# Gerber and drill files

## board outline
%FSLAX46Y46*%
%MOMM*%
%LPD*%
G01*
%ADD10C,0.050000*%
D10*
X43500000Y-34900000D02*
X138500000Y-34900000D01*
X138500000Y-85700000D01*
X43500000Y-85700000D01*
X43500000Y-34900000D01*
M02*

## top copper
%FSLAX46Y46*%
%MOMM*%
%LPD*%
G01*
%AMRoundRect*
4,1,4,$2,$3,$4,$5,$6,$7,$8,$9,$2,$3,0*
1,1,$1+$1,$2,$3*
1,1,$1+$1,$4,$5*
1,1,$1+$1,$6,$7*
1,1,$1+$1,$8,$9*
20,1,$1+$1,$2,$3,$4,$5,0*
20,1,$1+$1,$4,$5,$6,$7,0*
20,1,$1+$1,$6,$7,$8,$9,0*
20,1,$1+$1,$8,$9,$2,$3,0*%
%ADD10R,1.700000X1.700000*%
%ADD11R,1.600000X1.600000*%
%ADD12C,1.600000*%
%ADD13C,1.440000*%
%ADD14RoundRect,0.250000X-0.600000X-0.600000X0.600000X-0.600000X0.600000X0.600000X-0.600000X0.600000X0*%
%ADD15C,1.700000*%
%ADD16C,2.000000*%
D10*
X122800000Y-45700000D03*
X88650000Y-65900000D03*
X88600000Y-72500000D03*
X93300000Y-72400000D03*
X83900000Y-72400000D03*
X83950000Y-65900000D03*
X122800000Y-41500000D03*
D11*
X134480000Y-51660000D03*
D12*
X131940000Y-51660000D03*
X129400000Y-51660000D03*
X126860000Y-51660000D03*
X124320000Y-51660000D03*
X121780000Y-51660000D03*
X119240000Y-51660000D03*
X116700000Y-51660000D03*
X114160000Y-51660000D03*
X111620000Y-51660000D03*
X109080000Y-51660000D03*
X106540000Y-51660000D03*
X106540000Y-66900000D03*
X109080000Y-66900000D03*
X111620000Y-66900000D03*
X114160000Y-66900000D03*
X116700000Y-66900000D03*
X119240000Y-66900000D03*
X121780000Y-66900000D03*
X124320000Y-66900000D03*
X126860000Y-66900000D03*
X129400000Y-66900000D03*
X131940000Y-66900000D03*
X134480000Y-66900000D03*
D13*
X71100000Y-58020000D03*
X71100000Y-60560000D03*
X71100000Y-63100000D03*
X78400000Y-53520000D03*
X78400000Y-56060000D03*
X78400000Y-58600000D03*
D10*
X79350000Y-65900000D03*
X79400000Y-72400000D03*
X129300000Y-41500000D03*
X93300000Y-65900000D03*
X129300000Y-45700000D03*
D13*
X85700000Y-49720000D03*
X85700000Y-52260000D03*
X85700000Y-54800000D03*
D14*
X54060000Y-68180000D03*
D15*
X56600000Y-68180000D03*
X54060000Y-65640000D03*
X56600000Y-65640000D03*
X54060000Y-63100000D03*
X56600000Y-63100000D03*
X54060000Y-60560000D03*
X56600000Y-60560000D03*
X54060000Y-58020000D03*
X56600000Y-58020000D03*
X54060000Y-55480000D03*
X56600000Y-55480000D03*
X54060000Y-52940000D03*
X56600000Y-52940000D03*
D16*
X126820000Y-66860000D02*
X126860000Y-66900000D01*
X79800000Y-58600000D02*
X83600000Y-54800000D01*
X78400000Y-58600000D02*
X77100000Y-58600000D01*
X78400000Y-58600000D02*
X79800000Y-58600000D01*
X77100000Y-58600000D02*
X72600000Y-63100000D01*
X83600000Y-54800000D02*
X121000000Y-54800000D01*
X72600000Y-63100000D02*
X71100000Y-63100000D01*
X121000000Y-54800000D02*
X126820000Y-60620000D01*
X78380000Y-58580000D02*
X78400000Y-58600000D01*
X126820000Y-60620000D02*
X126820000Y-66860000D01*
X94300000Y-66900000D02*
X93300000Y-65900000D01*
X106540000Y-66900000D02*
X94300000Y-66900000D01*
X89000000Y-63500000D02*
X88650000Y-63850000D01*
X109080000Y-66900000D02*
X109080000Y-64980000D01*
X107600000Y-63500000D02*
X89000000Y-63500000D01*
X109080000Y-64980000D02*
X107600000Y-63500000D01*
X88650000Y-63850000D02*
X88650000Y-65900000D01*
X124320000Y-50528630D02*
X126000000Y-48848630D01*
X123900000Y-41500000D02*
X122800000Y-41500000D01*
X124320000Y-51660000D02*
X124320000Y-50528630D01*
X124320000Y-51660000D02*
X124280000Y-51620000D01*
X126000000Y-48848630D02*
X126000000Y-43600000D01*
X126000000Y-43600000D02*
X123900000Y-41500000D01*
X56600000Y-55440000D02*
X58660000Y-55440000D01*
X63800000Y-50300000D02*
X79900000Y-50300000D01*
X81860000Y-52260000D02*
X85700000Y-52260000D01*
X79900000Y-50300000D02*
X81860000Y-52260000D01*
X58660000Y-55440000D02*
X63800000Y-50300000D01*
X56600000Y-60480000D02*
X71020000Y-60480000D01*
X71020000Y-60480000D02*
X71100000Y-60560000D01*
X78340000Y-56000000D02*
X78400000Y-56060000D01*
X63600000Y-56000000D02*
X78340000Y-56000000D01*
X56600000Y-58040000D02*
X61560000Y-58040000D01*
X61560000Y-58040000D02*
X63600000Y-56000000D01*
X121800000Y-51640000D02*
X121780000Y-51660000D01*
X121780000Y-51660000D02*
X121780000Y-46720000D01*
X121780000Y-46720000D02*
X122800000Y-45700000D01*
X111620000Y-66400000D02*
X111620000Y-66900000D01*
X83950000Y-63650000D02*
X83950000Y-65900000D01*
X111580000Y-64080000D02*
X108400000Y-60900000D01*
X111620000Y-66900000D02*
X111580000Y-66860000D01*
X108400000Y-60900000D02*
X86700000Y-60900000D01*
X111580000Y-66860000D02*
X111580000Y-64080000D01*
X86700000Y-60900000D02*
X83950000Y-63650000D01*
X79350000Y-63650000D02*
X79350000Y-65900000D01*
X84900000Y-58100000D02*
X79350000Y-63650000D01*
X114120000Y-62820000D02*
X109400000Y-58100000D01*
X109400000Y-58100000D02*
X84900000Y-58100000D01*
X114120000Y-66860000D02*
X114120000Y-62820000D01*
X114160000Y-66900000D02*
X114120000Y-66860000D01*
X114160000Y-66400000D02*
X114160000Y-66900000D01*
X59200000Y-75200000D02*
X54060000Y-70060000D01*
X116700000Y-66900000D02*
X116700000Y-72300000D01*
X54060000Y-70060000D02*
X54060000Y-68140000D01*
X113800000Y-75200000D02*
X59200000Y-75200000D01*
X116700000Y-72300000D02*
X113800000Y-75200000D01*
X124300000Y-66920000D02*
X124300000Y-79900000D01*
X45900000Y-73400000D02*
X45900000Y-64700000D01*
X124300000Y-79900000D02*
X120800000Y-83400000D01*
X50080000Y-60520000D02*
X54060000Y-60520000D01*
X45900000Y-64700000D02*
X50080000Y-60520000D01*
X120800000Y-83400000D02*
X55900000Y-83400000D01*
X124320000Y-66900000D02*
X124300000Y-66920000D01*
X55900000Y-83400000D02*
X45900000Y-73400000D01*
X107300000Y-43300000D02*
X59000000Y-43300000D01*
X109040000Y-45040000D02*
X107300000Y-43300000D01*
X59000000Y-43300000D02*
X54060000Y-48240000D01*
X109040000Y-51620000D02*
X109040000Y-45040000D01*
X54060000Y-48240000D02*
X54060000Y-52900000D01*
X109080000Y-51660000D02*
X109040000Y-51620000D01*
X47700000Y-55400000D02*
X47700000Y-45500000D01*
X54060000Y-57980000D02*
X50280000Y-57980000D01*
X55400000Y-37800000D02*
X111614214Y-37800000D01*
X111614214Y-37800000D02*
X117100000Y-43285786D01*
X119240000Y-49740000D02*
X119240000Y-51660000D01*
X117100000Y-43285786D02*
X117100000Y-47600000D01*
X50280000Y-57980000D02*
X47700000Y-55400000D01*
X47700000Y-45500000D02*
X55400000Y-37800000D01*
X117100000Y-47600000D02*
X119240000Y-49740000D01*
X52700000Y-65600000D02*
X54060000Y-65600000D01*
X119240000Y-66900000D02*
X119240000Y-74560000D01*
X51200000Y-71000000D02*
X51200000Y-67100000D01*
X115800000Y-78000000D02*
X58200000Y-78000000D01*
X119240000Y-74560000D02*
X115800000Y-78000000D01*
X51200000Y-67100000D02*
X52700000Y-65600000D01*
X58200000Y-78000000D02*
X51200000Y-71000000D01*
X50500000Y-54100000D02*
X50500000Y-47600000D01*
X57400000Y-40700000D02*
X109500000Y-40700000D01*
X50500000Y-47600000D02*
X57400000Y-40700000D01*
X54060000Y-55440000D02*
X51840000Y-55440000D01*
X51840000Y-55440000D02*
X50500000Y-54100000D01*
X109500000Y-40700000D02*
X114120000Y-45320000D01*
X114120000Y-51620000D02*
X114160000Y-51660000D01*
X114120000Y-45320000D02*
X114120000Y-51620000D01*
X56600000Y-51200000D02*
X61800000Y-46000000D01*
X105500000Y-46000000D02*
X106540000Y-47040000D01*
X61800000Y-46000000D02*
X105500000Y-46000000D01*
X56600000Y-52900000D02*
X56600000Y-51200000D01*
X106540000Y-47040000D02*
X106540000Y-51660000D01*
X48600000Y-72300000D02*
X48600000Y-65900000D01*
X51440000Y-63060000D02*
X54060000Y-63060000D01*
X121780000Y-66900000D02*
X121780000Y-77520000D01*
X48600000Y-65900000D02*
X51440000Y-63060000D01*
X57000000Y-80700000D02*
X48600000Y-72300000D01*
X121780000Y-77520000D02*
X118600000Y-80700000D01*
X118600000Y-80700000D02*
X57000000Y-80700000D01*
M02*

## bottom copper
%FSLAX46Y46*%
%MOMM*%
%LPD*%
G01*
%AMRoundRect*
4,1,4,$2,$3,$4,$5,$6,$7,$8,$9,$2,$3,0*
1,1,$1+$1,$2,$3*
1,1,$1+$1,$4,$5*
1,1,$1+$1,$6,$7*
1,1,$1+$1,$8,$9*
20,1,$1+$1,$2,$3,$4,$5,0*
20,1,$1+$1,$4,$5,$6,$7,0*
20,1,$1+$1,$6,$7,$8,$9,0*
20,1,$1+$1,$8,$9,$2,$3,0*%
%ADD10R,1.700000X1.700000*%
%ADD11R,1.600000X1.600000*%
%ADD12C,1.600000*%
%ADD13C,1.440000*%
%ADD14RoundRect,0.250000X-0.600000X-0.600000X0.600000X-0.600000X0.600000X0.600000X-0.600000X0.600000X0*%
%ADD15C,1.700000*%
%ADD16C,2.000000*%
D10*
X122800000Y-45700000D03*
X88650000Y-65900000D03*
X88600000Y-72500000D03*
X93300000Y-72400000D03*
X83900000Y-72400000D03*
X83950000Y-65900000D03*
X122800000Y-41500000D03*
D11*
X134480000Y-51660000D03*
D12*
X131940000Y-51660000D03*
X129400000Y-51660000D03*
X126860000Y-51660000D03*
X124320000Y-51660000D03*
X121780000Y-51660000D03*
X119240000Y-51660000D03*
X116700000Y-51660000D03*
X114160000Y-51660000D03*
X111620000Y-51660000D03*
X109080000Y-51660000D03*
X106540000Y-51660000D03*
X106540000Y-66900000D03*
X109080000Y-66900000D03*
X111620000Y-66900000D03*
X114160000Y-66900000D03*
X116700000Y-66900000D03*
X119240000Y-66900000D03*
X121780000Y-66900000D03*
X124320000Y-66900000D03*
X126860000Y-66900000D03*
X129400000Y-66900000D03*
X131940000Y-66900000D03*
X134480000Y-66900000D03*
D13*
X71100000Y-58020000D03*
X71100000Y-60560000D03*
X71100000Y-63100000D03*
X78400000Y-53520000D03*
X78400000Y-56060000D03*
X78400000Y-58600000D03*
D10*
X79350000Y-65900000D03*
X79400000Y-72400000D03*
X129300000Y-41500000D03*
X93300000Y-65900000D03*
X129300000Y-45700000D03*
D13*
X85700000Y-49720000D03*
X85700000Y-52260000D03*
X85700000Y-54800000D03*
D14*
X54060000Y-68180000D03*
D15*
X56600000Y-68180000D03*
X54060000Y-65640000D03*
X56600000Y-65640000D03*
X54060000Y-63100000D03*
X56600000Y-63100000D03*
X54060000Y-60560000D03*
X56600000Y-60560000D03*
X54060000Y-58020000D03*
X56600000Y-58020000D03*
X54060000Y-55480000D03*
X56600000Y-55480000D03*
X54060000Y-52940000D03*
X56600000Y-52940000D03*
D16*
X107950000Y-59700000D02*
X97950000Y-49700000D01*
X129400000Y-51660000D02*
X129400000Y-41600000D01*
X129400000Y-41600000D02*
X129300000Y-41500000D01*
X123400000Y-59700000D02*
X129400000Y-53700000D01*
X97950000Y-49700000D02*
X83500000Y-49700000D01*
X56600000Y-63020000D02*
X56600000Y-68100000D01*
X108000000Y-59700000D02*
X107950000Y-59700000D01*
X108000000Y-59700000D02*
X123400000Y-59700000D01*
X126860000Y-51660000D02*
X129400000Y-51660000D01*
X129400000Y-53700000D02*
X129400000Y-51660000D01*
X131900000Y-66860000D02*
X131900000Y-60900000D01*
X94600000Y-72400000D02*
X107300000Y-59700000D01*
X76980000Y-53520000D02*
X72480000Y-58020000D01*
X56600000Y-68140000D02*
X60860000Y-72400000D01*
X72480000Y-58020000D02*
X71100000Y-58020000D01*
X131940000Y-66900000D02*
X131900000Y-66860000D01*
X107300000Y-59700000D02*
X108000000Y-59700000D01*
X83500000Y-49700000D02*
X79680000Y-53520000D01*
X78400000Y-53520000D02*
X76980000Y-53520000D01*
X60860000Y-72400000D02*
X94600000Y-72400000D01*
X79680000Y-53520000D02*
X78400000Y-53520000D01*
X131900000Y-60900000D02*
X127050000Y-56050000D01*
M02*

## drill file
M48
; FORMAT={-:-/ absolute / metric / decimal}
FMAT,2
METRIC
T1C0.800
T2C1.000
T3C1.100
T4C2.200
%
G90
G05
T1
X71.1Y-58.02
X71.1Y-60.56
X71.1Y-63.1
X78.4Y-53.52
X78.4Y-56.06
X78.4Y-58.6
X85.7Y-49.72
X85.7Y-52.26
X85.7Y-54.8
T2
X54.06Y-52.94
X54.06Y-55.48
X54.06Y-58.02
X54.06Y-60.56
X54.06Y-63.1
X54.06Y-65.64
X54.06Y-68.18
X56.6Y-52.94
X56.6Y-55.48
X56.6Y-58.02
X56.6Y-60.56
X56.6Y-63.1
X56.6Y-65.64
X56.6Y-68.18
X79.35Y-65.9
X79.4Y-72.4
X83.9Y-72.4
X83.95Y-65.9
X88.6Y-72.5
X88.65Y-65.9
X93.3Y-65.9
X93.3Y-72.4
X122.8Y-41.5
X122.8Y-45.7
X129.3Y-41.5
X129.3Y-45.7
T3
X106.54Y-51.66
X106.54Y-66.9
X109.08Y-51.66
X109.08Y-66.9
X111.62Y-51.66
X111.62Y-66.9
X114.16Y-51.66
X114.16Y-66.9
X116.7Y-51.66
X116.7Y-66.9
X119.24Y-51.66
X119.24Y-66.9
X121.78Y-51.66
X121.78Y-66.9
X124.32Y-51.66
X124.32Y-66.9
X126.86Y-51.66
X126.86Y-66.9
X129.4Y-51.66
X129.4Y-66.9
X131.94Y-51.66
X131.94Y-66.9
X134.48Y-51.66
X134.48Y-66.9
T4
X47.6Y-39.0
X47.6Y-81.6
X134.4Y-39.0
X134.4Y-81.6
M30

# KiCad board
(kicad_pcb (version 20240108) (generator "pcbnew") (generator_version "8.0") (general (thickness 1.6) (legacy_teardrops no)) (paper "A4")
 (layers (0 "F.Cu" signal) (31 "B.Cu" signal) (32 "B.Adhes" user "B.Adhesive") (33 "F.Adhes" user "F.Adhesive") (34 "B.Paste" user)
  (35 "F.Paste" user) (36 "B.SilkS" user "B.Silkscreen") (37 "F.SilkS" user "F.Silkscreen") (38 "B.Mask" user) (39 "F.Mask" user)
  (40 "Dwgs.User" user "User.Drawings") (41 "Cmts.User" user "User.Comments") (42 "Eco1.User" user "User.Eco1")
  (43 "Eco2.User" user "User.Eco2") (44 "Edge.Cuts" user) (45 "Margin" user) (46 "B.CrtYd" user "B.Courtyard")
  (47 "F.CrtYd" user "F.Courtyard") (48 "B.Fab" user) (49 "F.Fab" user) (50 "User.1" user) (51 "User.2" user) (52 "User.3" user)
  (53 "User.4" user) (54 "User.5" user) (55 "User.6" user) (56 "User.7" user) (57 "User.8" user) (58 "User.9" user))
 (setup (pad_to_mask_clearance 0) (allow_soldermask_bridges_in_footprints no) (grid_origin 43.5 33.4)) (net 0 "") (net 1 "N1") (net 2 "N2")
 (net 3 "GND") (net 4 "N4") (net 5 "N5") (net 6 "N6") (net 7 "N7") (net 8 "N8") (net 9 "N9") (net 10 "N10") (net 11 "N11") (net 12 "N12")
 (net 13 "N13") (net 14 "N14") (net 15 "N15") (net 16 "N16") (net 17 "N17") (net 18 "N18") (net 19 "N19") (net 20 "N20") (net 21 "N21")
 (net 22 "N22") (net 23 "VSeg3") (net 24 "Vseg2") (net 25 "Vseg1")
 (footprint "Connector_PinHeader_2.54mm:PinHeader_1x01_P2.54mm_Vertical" (layer "F.Cu") (at 122.8 45.7 180)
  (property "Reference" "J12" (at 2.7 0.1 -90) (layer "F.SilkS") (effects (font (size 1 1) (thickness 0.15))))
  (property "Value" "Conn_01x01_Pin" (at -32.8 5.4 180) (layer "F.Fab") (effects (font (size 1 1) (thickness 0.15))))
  (pad "1" thru_hole rect (at 0 0 180) (size 1.7 1.7) (drill 1) (layers "*.Cu" "*.Mask") (remove_unused_layers no) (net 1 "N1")))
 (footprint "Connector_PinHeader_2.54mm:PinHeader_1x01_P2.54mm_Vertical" (layer "F.Cu") (at 88.65 65.9 180)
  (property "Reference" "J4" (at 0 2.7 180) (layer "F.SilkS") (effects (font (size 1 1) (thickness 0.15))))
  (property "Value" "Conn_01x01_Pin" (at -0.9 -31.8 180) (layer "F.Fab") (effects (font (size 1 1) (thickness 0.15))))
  (pad "1" thru_hole rect (at 0 0 180) (size 1.7 1.7) (drill 1) (layers "*.Cu" "*.Mask") (remove_unused_layers no) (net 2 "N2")))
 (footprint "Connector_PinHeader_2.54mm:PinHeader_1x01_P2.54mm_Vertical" (layer "F.Cu") (at 88.6 72.5 180)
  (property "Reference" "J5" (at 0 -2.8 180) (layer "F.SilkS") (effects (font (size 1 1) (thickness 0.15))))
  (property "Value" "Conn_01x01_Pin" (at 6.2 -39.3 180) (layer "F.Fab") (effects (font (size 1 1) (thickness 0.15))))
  (pad "1" thru_hole rect (at 0 0 180) (size 1.7 1.7) (drill 1) (layers "*.Cu" "*.Mask") (remove_unused_layers no) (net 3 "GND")))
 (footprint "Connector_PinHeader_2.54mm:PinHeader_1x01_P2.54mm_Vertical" (layer "F.Cu") (at 93.3 72.4 180)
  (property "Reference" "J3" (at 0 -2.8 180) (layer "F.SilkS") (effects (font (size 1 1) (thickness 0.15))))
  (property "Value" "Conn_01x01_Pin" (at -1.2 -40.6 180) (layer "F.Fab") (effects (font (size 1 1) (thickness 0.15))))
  (pad "1" thru_hole rect (at 0 0 180) (size 1.7 1.7) (drill 1) (layers "*.Cu" "*.Mask") (remove_unused_layers no) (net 3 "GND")))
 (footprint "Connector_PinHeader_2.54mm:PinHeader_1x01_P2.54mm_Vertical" (layer "F.Cu") (at 83.9 72.4 180)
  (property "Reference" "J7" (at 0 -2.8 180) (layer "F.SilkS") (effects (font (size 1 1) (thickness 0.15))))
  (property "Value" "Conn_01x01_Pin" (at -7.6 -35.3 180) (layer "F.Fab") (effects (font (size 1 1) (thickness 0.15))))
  (pad "1" thru_hole rect (at 0 0 180) (size 1.7 1.7) (drill 1) (layers "*.Cu" "*.Mask") (remove_unused_layers no) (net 3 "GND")))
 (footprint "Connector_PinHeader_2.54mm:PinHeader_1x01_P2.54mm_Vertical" (layer "F.Cu") (at 83.95 65.9 180)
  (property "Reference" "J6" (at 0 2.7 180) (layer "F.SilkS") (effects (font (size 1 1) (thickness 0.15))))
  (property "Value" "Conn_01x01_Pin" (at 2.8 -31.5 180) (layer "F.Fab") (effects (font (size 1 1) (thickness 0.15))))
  (pad "1" thru_hole rect (at 0 0 180) (size 1.7 1.7) (drill 1) (layers "*.Cu" "*.Mask") (remove_unused_layers no) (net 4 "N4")))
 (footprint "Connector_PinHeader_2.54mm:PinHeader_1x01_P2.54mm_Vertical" (layer "F.Cu") (at 122.8 41.5 180)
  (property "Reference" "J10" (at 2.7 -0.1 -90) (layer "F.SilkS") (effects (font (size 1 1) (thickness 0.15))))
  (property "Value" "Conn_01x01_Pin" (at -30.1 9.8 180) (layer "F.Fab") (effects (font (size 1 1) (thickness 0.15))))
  (pad "1" thru_hole rect (at 0 0 180) (size 1.7 1.7) (drill 1) (layers "*.Cu" "*.Mask") (remove_unused_layers no) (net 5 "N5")))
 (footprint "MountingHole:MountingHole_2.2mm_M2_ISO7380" (layer "F.Cu") (at 47.6 81.6)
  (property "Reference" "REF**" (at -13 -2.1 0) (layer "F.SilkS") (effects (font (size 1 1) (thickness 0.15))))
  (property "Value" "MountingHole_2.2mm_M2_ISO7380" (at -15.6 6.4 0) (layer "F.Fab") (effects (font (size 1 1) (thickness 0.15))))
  (pad "" np_thru_hole circle (at 0 0) (size 2.2 2.2) (drill 2.2) (layers "*.Cu" "*.Mask")))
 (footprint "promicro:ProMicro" (layer "F.Cu") (at 120.51 59.28 180)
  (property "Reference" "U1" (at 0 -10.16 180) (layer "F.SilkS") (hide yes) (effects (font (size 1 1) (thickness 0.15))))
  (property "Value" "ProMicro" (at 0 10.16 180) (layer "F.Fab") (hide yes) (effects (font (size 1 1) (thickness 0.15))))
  (pad "1" thru_hole rect (at -13.97 7.62 180) (size 1.6 1.6) (drill 1.1) (layers "*.Cu" "*.Mask" "F.SilkS") (remove_unused_layers no)
   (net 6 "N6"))
  (pad "2" thru_hole circle (at -11.43 7.62 180) (size 1.6 1.6) (drill 1.1) (layers "*.Cu" "*.Mask" "F.SilkS") (remove_unused_layers no)
   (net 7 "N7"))
  (pad "3" thru_hole circle (at -8.89 7.62 180) (size 1.6 1.6) (drill 1.1) (layers "*.Cu" "*.Mask" "F.SilkS") (remove_unused_layers no)
   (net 3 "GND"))
  (pad "4" thru_hole circle (at -6.35 7.62 180) (size 1.6 1.6) (drill 1.1) (layers "*.Cu" "*.Mask" "F.SilkS") (remove_unused_layers no)
   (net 3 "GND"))
  (pad "5" thru_hole circle (at -3.81 7.62 180) (size 1.6 1.6) (drill 1.1) (layers "*.Cu" "*.Mask" "F.SilkS") (remove_unused_layers no)
   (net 5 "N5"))
  (pad "6" thru_hole circle (at -1.27 7.62 180) (size 1.6 1.6) (drill 1.1) (layers "*.Cu" "*.Mask" "F.SilkS") (remove_unused_layers no)
   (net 1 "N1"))
  (pad "7" thru_hole circle (at 1.27 7.62 180) (size 1.6 1.6) (drill 1.1) (layers "*.Cu" "*.Mask" "F.SilkS") (remove_unused_layers no)
   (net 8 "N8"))
  (pad "8" thru_hole circle (at 3.81 7.62 180) (size 1.6 1.6) (drill 1.1) (layers "*.Cu" "*.Mask" "F.SilkS") (remove_unused_layers no)
   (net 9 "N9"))
  (pad "9" thru_hole circle (at 6.35 7.62 180) (size 1.6 1.6) (drill 1.1) (layers "*.Cu" "*.Mask" "F.SilkS") (remove_unused_layers no)
   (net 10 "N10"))
  (pad "10" thru_hole circle (at 8.89 7.62 180) (size 1.6 1.6) (drill 1.1) (layers "*.Cu" "*.Mask" "F.SilkS") (remove_unused_layers no)
   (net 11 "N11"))
  (pad "11" thru_hole circle (at 11.43 7.62 180) (size 1.6 1.6) (drill 1.1) (layers "*.Cu" "*.Mask" "F.SilkS") (remove_unused_layers no)
   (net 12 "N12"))
  (pad "12" thru_hole circle (at 13.97 7.62 180) (size 1.6 1.6) (drill 1.1) (layers "*.Cu" "*.Mask" "F.SilkS") (remove_unused_layers no)
   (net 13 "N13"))
  (pad "13" thru_hole circle (at 13.97 -7.62 180) (size 1.6 1.6) (drill 1.1) (layers "*.Cu" "*.Mask" "F.SilkS") (remove_unused_layers no)
   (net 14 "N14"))
  (pad "14" thru_hole circle (at 11.43 -7.62 180) (size 1.6 1.6) (drill 1.1) (layers "*.Cu" "*.Mask" "F.SilkS") (remove_unused_layers no)
   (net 2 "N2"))
  (pad "15" thru_hole circle (at 8.89 -7.62 180) (size 1.6 1.6) (drill 1.1) (layers "*.Cu" "*.Mask" "F.SilkS") (remove_unused_layers no)
   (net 4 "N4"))
  (pad "16" thru_hole circle (at 6.35 -7.62 180) (size 1.6 1.6) (drill 1.1) (layers "*.Cu" "*.Mask" "F.SilkS") (remove_unused_layers no)
   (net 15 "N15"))
  (pad "17" thru_hole circle (at 3.81 -7.62 180) (size 1.6 1.6) (drill 1.1) (layers "*.Cu" "*.Mask" "F.SilkS") (remove_unused_layers no)
   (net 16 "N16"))
  (pad "18" thru_hole circle (at 1.27 -7.62 180) (size 1.6 1.6) (drill 1.1) (layers "*.Cu" "*.Mask" "F.SilkS") (remove_unused_layers no)
   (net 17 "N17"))
  (pad "19" thru_hole circle (at -1.27 -7.62 180) (size 1.6 1.6) (drill 1.1) (layers "*.Cu" "*.Mask" "F.SilkS") (remove_unused_layers no)
   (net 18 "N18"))
  (pad "20" thru_hole circle (at -3.81 -7.62 180) (size 1.6 1.6) (drill 1.1) (layers "*.Cu" "*.Mask" "F.SilkS") (remove_unused_layers no)
   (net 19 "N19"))
  (pad "21" thru_hole circle (at -6.35 -7.62 180) (size 1.6 1.6) (drill 1.1) (layers "*.Cu" "*.Mask" "F.SilkS") (remove_unused_layers no)
   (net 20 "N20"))
  (pad "22" thru_hole circle (at -8.89 -7.62 180) (size 1.6 1.6) (drill 1.1) (layers "*.Cu" "*.Mask" "F.SilkS") (remove_unused_layers no)
   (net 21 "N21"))
  (pad "23" thru_hole circle (at -11.43 -7.62 180) (size 1.6 1.6) (drill 1.1) (layers "*.Cu" "*.Mask" "F.SilkS") (remove_unused_layers no)
   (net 3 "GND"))
  (pad "24" thru_hole circle (at -13.97 -7.62 180) (size 1.6 1.6) (drill 1.1) (layers "*.Cu" "*.Mask" "F.SilkS") (remove_unused_layers no)
   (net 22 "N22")))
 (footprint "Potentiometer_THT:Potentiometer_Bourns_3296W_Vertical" (layer "F.Cu") (at 71.1 58.02 90)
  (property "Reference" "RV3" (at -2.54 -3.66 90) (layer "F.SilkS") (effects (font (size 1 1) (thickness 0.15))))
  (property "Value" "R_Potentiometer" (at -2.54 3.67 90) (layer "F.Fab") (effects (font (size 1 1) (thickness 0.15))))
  (pad "1" thru_hole circle (at 0 0 90) (size 1.44 1.44) (drill 0.8) (layers "*.Cu" "*.Mask") (remove_unused_layers no) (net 3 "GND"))
  (pad "2" thru_hole circle (at -2.54 0 90) (size 1.44 1.44) (drill 0.8) (layers "*.Cu" "*.Mask") (remove_unused_layers no) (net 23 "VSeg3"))
  (pad "3" thru_hole circle (at -5.08 0 90) (size 1.44 1.44) (drill 0.8) (layers "*.Cu" "*.Mask") (remove_unused_layers no) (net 20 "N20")))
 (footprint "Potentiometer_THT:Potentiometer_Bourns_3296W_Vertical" (layer "F.Cu") (at 78.4 53.52 90)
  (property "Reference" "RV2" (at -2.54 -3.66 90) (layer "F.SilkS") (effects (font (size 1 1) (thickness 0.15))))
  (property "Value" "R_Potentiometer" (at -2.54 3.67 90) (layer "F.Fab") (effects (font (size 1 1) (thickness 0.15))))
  (pad "1" thru_hole circle (at 0 0 90) (size 1.44 1.44) (drill 0.8) (layers "*.Cu" "*.Mask") (remove_unused_layers no) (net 3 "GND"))
  (pad "2" thru_hole circle (at -2.54 0 90) (size 1.44 1.44) (drill 0.8) (layers "*.Cu" "*.Mask") (remove_unused_layers no) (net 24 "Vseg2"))
  (pad "3" thru_hole circle (at -5.08 0 90) (size 1.44 1.44) (drill 0.8) (layers "*.Cu" "*.Mask") (remove_unused_layers no) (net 20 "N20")))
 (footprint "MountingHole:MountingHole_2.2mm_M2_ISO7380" (layer "F.Cu") (at 47.6 39)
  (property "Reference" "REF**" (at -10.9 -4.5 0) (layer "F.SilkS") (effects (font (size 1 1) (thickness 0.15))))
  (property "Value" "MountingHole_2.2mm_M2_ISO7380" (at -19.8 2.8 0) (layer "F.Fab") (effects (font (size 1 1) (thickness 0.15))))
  (pad "" np_thru_hole circle (at 0 0) (size 2.2 2.2) (drill 2.2) (layers "*.Cu" "*.Mask")))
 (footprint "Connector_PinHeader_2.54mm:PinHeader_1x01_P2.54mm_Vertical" (layer "F.Cu") (at 79.35 65.9 180)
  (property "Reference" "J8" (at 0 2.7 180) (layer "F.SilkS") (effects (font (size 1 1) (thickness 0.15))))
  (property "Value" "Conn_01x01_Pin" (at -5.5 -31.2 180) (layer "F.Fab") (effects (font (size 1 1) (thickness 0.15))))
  (pad "1" thru_hole rect (at 0 0 180) (size 1.7 1.7) (drill 1) (layers "*.Cu" "*.Mask") (remove_unused_layers no) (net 15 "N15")))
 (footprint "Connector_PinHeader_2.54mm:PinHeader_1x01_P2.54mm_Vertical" (layer "F.Cu") (at 79.4 72.4 180)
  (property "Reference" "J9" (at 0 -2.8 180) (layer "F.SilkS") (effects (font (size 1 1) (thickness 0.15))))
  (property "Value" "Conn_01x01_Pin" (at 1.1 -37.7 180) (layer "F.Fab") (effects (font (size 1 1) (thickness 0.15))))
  (pad "1" thru_hole rect (at 0 0 180) (size 1.7 1.7) (drill 1) (layers "*.Cu" "*.Mask") (remove_unused_layers no) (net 3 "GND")))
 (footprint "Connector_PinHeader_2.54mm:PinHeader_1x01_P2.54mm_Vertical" (layer "F.Cu") (at 129.3 41.5 180)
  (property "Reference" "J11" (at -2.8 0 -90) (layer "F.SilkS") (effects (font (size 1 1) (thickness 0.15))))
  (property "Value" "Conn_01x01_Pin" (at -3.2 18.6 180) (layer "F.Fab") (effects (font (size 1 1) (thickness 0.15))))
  (pad "1" thru_hole rect (at 0 0 180) (size 1.7 1.7) (drill 1) (layers "*.Cu" "*.Mask") (remove_unused_layers no) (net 3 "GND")))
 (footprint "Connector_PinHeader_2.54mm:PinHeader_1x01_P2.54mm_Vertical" (layer "F.Cu") (at 93.3 65.9 180)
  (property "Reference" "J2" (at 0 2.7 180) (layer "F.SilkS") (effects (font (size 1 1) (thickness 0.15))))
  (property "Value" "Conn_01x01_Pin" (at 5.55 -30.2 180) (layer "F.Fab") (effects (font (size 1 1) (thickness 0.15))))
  (pad "1" thru_hole rect (at 0 0 180) (size 1.7 1.7) (drill 1) (layers "*.Cu" "*.Mask") (remove_unused_layers no) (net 14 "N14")))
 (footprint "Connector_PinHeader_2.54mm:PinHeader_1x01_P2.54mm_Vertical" (layer "F.Cu") (at 129.3 45.7 180)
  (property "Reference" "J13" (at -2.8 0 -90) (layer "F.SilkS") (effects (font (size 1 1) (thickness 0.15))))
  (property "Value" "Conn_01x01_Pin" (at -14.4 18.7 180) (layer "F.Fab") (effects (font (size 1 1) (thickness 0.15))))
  (pad "1" thru_hole rect (at 0 0 180) (size 1.7 1.7) (drill 1) (layers "*.Cu" "*.Mask") (remove_unused_layers no) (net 3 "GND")))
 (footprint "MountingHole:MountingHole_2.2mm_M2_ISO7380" (layer "F.Cu") (at 134.4 81.6)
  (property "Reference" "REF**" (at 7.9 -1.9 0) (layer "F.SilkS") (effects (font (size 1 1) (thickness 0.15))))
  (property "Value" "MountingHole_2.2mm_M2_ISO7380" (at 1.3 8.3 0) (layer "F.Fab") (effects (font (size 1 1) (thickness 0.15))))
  (pad "" np_thru_hole circle (at 0 0) (size 2.2 2.2) (drill 2.2) (layers "*.Cu" "*.Mask")))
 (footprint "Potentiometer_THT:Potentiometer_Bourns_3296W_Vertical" (layer "F.Cu") (at 85.7 49.72 90)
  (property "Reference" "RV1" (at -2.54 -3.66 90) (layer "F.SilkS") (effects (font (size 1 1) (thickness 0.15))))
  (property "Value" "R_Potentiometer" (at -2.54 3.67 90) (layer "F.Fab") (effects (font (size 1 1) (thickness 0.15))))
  (pad "1" thru_hole circle (at 0 0 90) (size 1.44 1.44) (drill 0.8) (layers "*.Cu" "*.Mask") (remove_unused_layers no) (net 3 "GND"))
  (pad "2" thru_hole circle (at -2.54 0 90) (size 1.44 1.44) (drill 0.8) (layers "*.Cu" "*.Mask") (remove_unused_layers no) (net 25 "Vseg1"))
  (pad "3" thru_hole circle (at -5.08 0 90) (size 1.44 1.44) (drill 0.8) (layers "*.Cu" "*.Mask") (remove_unused_layers no) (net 20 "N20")))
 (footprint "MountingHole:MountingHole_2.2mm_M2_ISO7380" (layer "F.Cu") (at 134.4 39)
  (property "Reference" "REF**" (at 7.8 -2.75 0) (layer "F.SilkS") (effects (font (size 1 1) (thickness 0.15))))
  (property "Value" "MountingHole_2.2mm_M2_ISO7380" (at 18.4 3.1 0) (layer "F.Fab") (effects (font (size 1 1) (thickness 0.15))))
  (pad "" np_thru_hole circle (at 0 0) (size 2.2 2.2) (drill 2.2) (layers "*.Cu" "*.Mask")))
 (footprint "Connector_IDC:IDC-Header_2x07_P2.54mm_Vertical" (layer "B.Cu") (at 54.06 68.18)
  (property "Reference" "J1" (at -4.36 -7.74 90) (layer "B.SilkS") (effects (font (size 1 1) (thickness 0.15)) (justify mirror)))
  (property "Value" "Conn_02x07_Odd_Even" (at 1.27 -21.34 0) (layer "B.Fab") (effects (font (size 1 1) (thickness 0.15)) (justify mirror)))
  (pad "1" thru_hole roundrect (at 0 0) (size 1.7 1.7) (drill 1) (layers "*.Cu" "*.Mask") (remove_unused_layers no)
   (roundrect_rratio 0.147059) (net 16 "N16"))
  (pad "2" thru_hole circle (at 2.54 0) (size 1.7 1.7) (drill 1) (layers "*.Cu" "*.Mask") (remove_unused_layers no) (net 3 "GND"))
  (pad "3" thru_hole circle (at 0 -2.54) (size 1.7 1.7) (drill 1) (layers "*.Cu" "*.Mask") (remove_unused_layers no) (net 17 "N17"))
  (pad "4" thru_hole circle (at 2.54 -2.54) (size 1.7 1.7) (drill 1) (layers "*.Cu" "*.Mask") (remove_unused_layers no) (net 3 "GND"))
  (pad "5" thru_hole circle (at 0 -5.08) (size 1.7 1.7) (drill 1) (layers "*.Cu" "*.Mask") (remove_unused_layers no) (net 18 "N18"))
  (pad "6" thru_hole circle (at 2.54 -5.08) (size 1.7 1.7) (drill 1) (layers "*.Cu" "*.Mask") (remove_unused_layers no) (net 3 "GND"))
  (pad "7" thru_hole circle (at 0 -7.62) (size 1.7 1.7) (drill 1) (layers "*.Cu" "*.Mask") (remove_unused_layers no) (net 19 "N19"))
  (pad "8" thru_hole circle (at 2.54 -7.62) (size 1.7 1.7) (drill 1) (layers "*.Cu" "*.Mask") (remove_unused_layers no) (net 23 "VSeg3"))
  (pad "9" thru_hole circle (at 0 -10.16) (size 1.7 1.7) (drill 1) (layers "*.Cu" "*.Mask") (remove_unused_layers no) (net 8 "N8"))
  (pad "10" thru_hole circle (at 2.54 -10.16) (size 1.7 1.7) (drill 1) (layers "*.Cu" "*.Mask") (remove_unused_layers no) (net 24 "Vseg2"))
  (pad "11" thru_hole circle (at 0 -12.7) (size 1.7 1.7) (drill 1) (layers "*.Cu" "*.Mask") (remove_unused_layers no) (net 10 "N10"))
  (pad "12" thru_hole circle (at 2.54 -12.7) (size 1.7 1.7) (drill 1) (layers "*.Cu" "*.Mask") (remove_unused_layers no) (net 25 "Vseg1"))
  (pad "13" thru_hole circle (at 0 -15.24) (size 1.7 1.7) (drill 1) (layers "*.Cu" "*.Mask") (remove_unused_layers no) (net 12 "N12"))
  (pad "14" thru_hole circle (at 2.54 -15.24) (size 1.7 1.7) (drill 1) (layers "*.Cu" "*.Mask") (remove_unused_layers no) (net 13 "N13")))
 (gr_rect (start 43.5 34.9) (end 138.5 85.7) (stroke (width 0.05) (type default)) (fill none) (layer "Edge.Cuts"))
 (segment (start 126.82 66.86) (end 126.86 66.9) (width 2) (layer "F.Cu") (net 20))
 (segment (start 79.8 58.6) (end 83.6 54.8) (width 2) (layer "F.Cu") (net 20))
 (segment (start 78.4 58.6) (end 77.1 58.6) (width 2) (layer "F.Cu") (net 20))
 (segment (start 78.4 58.6) (end 79.8 58.6) (width 2) (layer "F.Cu") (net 20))
 (segment (start 77.1 58.6) (end 72.6 63.1) (width 2) (layer "F.Cu") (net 20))
 (segment (start 83.6 54.8) (end 121 54.8) (width 2) (layer "F.Cu") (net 20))
 (segment (start 72.6 63.1) (end 71.1 63.1) (width 2) (layer "F.Cu") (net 20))
 (segment (start 121 54.8) (end 126.82 60.62) (width 2) (layer "F.Cu") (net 20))
 (segment (start 78.38 58.58) (end 78.4 58.6) (width 2) (layer "F.Cu") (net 20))
 (segment (start 126.82 60.62) (end 126.82 66.86) (width 2) (layer "F.Cu") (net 20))
 (segment (start 94.3 66.9) (end 93.3 65.9) (width 2) (layer "F.Cu") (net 14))
 (segment (start 106.54 66.9) (end 94.3 66.9) (width 2) (layer "F.Cu") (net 14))
 (segment (start 89 63.5) (end 88.65 63.85) (width 2) (layer "F.Cu") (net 2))
 (segment (start 109.08 66.9) (end 109.08 64.98) (width 2) (layer "F.Cu") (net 2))
 (segment (start 107.6 63.5) (end 89 63.5) (width 2) (layer "F.Cu") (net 2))
 (segment (start 109.08 64.98) (end 107.6 63.5) (width 2) (layer "F.Cu") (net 2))
 (segment (start 88.65 63.85) (end 88.65 65.9) (width 2) (layer "F.Cu") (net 2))
 (segment (start 124.32 50.52863) (end 126 48.84863) (width 2) (layer "F.Cu") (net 5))
 (segment (start 123.9 41.5) (end 122.8 41.5) (width 2) (layer "F.Cu") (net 5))
 (segment (start 124.32 51.66) (end 124.32 50.52863) (width 2) (layer "F.Cu") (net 5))
 (segment (start 124.32 51.66) (end 124.28 51.62) (width 2) (layer "F.Cu") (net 5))
 (segment (start 126 48.84863) (end 126 43.6) (width 2) (layer "F.Cu") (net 5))
 (segment (start 126 43.6) (end 123.9 41.5) (width 2) (layer "F.Cu") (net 5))
 (segment (start 56.6 55.44) (end 58.66 55.44) (width 2) (layer "F.Cu") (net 25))
 (segment (start 63.8 50.3) (end 79.9 50.3) (width 2) (layer "F.Cu") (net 25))
 (segment (start 81.86 52.26) (end 85.7 52.26) (width 2) (layer "F.Cu") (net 25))
 (segment (start 79.9 50.3) (end 81.86 52.26) (width 2) (layer "F.Cu") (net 25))
 (segment (start 58.66 55.44) (end 63.8 50.3) (width 2) (layer "F.Cu") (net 25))
 (segment (start 56.6 60.48) (end 71.02 60.48) (width 2) (layer "F.Cu") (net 23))
 (segment (start 71.02 60.48) (end 71.1 60.56) (width 2) (layer "F.Cu") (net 23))
 (segment (start 107.95 59.7) (end 97.95 49.7) (width 2) (layer "B.Cu") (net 3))
 (segment (start 129.4 51.66) (end 129.4 41.6) (width 2) (layer "B.Cu") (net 3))
 (segment (start 129.4 41.6) (end 129.3 41.5) (width 2) (layer "B.Cu") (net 3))
 (segment (start 123.4 59.7) (end 129.4 53.7) (width 2) (layer "B.Cu") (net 3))
 (segment (start 97.95 49.7) (end 83.5 49.7) (width 2) (layer "B.Cu") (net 3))
 (segment (start 56.6 63.02) (end 56.6 68.1) (width 2) (layer "B.Cu") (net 3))
 (segment (start 108 59.7) (end 107.95 59.7) (width 2) (layer "B.Cu") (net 3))
 (segment (start 108 59.7) (end 123.4 59.7) (width 2) (layer "B.Cu") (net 3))
 (segment (start 126.86 51.66) (end 129.4 51.66) (width 2) (layer "B.Cu") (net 3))
 (segment (start 129.4 53.7) (end 129.4 51.66) (width 2) (layer "B.Cu") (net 3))
 (segment (start 131.9 66.86) (end 131.9 60.9) (width 2) (layer "B.Cu") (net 3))
 (segment (start 94.6 72.4) (end 107.3 59.7) (width 2) (layer "B.Cu") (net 3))
 (segment (start 76.98 53.52) (end 72.48 58.02) (width 2) (layer "B.Cu") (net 3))
 (segment (start 56.6 68.14) (end 60.86 72.4) (width 2) (layer "B.Cu") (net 3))
 (segment (start 72.48 58.02) (end 71.1 58.02) (width 2) (layer "B.Cu") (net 3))
 (segment (start 131.94 66.9) (end 131.9 66.86) (width 2) (layer "B.Cu") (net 3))
 (segment (start 107.3 59.7) (end 108 59.7) (width 2) (layer "B.Cu") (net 3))
 (segment (start 83.5 49.7) (end 79.68 53.52) (width 2) (layer "B.Cu") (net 3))
 (segment (start 78.4 53.52) (end 76.98 53.52) (width 2) (layer "B.Cu") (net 3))
 (segment (start 60.86 72.4) (end 94.6 72.4) (width 2) (layer "B.Cu") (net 3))
 (segment (start 79.68 53.52) (end 78.4 53.52) (width 2) (layer "B.Cu") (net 3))
 (segment (start 131.9 60.9) (end 127.05 56.05) (width 2) (layer "B.Cu") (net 3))
 (segment (start 78.34 56) (end 78.4 56.06) (width 2) (layer "F.Cu") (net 24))
 (segment (start 63.6 56) (end 78.34 56) (width 2) (layer "F.Cu") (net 24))
 (segment (start 56.6 58.04) (end 61.56 58.04) (width 2) (layer "F.Cu") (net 24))
 (segment (start 61.56 58.04) (end 63.6 56) (width 2) (layer "F.Cu") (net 24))
 (segment (start 121.8 51.64) (end 121.78 51.66) (width 2) (layer "F.Cu") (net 1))
 (segment (start 121.78 51.66) (end 121.78 46.72) (width 2) (layer "F.Cu") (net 1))
 (segment (start 121.78 46.72) (end 122.8 45.7) (width 2) (layer "F.Cu") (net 1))
 (segment (start 111.62 66.4) (end 111.62 66.9) (width 2) (layer "F.Cu") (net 4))
 (segment (start 83.95 63.65) (end 83.95 65.9) (width 2) (layer "F.Cu") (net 4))
 (segment (start 111.58 64.08) (end 108.4 60.9) (width 2) (layer "F.Cu") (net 4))
 (segment (start 111.62 66.9) (end 111.58 66.86) (width 2) (layer "F.Cu") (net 4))
 (segment (start 108.4 60.9) (end 86.7 60.9) (width 2) (layer "F.Cu") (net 4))
 (segment (start 111.58 66.86) (end 111.58 64.08) (width 2) (layer "F.Cu") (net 4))
 (segment (start 86.7 60.9) (end 83.95 63.65) (width 2) (layer "F.Cu") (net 4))
 (segment (start 79.35 63.65) (end 79.35 65.9) (width 2) (layer "F.Cu") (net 15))
 (segment (start 84.9 58.1) (end 79.35 63.65) (width 2) (layer "F.Cu") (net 15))
 (segment (start 114.12 62.82) (end 109.4 58.1) (width 2) (layer "F.Cu") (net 15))
 (segment (start 109.4 58.1) (end 84.9 58.1) (width 2) (layer "F.Cu") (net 15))
 (segment (start 114.12 66.86) (end 114.12 62.82) (width 2) (layer "F.Cu") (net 15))
 (segment (start 114.16 66.9) (end 114.12 66.86) (width 2) (layer "F.Cu") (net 15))
 (segment (start 114.16 66.4) (end 114.16 66.9) (width 2) (layer "F.Cu") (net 15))
 (segment (start 59.2 75.2) (end 54.06 70.06) (width 2) (layer "F.Cu") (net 16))
 (segment (start 116.7 66.9) (end 116.7 72.3) (width 2) (layer "F.Cu") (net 16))
 (segment (start 54.06 70.06) (end 54.06 68.14) (width 2) (layer "F.Cu") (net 16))
 (segment (start 113.8 75.2) (end 59.2 75.2) (width 2) (layer "F.Cu") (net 16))
 (segment (start 116.7 72.3) (end 113.8 75.2) (width 2) (layer "F.Cu") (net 16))
 (segment (start 124.3 66.92) (end 124.3 79.9) (width 2) (layer "F.Cu") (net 19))
 (segment (start 45.9 73.4) (end 45.9 64.7) (width 2) (layer "F.Cu") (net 19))
 (segment (start 124.3 79.9) (end 120.8 83.4) (width 2) (layer "F.Cu") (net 19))
 (segment (start 50.08 60.52) (end 54.06 60.52) (width 2) (layer "F.Cu") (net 19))
 (segment (start 45.9 64.7) (end 50.08 60.52) (width 2) (layer "F.Cu") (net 19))
 (segment (start 120.8 83.4) (end 55.9 83.4) (width 2) (layer "F.Cu") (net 19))
 (segment (start 124.32 66.9) (end 124.3 66.92) (width 2) (layer "F.Cu") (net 19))
 (segment (start 55.9 83.4) (end 45.9 73.4) (width 2) (layer "F.Cu") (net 19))
 (segment (start 107.3 43.3) (end 59 43.3) (width 2) (layer "F.Cu") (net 12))
 (segment (start 109.04 45.04) (end 107.3 43.3) (width 2) (layer "F.Cu") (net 12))
 (segment (start 59 43.3) (end 54.06 48.24) (width 2) (layer "F.Cu") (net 12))
 (segment (start 109.04 51.62) (end 109.04 45.04) (width 2) (layer "F.Cu") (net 12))
 (segment (start 54.06 48.24) (end 54.06 52.9) (width 2) (layer "F.Cu") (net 12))
 (segment (start 109.08 51.66) (end 109.04 51.62) (width 2) (layer "F.Cu") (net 12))
 (segment (start 47.7 55.4) (end 47.7 45.5) (width 2) (layer "F.Cu") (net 8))
 (segment (start 54.06 57.98) (end 50.28 57.98) (width 2) (layer "F.Cu") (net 8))
 (segment (start 55.4 37.8) (end 111.614214 37.8) (width 2) (layer "F.Cu") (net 8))
 (segment (start 111.614214 37.8) (end 117.1 43.285786) (width 2) (layer "F.Cu") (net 8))
 (segment (start 119.24 49.74) (end 119.24 51.66) (width 2) (layer "F.Cu") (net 8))
 (segment (start 117.1 43.285786) (end 117.1 47.6) (width 2) (layer "F.Cu") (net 8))
 (segment (start 50.28 57.98) (end 47.7 55.4) (width 2) (layer "F.Cu") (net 8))
 (segment (start 47.7 45.5) (end 55.4 37.8) (width 2) (layer "F.Cu") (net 8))
 (segment (start 117.1 47.6) (end 119.24 49.74) (width 2) (layer "F.Cu") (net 8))
 (segment (start 52.7 65.6) (end 54.06 65.6) (width 2) (layer "F.Cu") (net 17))
 (segment (start 119.24 66.9) (end 119.24 74.56) (width 2) (layer "F.Cu") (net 17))
 (segment (start 51.2 71) (end 51.2 67.1) (width 2) (layer "F.Cu") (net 17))
 (segment (start 115.8 78) (end 58.2 78) (width 2) (layer "F.Cu") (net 17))
 (segment (start 119.24 74.56) (end 115.8 78) (width 2) (layer "F.Cu") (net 17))
 (segment (start 51.2 67.1) (end 52.7 65.6) (width 2) (layer "F.Cu") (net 17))
 (segment (start 58.2 78) (end 51.2 71) (width 2) (layer "F.Cu") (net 17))
 (segment (start 50.5 54.1) (end 50.5 47.6) (width 2) (layer "F.Cu") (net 10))
 (segment (start 57.4 40.7) (end 109.5 40.7) (width 2) (layer "F.Cu") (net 10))
 (segment (start 50.5 47.6) (end 57.4 40.7) (width 2) (layer "F.Cu") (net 10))
 (segment (start 54.06 55.44) (end 51.84 55.44) (width 2) (layer "F.Cu") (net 10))
 (segment (start 51.84 55.44) (end 50.5 54.1) (width 2) (layer "F.Cu") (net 10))
 (segment (start 109.5 40.7) (end 114.12 45.32) (width 2) (layer "F.Cu") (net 10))
 (segment (start 114.12 51.62) (end 114.16 51.66) (width 2) (layer "F.Cu") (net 10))
 (segment (start 114.12 45.32) (end 114.12 51.62) (width 2) (layer "F.Cu") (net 10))
 (segment (start 56.6 51.2) (end 61.8 46) (width 2) (layer "F.Cu") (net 13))
 (segment (start 105.5 46) (end 106.54 47.04) (width 2) (layer "F.Cu") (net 13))
 (segment (start 61.8 46) (end 105.5 46) (width 2) (layer "F.Cu") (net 13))
 (segment (start 56.6 52.9) (end 56.6 51.2) (width 2) (layer "F.Cu") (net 13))
 (segment (start 106.54 47.04) (end 106.54 51.66) (width 2) (layer "F.Cu") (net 13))
 (segment (start 48.6 72.3) (end 48.6 65.9) (width 2) (layer "F.Cu") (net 18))
 (segment (start 51.44 63.06) (end 54.06 63.06) (width 2) (layer "F.Cu") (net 18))
 (segment (start 121.78 66.9) (end 121.78 77.52) (width 2) (layer "F.Cu") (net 18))
 (segment (start 48.6 65.9) (end 51.44 63.06) (width 2) (layer "F.Cu") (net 18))
 (segment (start 57 80.7) (end 48.6 72.3) (width 2) (layer "F.Cu") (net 18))
 (segment (start 121.78 77.52) (end 118.6 80.7) (width 2) (layer "F.Cu") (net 18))
 (segment (start 118.6 80.7) (end 57 80.7) (width 2) (layer "F.Cu") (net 18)))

